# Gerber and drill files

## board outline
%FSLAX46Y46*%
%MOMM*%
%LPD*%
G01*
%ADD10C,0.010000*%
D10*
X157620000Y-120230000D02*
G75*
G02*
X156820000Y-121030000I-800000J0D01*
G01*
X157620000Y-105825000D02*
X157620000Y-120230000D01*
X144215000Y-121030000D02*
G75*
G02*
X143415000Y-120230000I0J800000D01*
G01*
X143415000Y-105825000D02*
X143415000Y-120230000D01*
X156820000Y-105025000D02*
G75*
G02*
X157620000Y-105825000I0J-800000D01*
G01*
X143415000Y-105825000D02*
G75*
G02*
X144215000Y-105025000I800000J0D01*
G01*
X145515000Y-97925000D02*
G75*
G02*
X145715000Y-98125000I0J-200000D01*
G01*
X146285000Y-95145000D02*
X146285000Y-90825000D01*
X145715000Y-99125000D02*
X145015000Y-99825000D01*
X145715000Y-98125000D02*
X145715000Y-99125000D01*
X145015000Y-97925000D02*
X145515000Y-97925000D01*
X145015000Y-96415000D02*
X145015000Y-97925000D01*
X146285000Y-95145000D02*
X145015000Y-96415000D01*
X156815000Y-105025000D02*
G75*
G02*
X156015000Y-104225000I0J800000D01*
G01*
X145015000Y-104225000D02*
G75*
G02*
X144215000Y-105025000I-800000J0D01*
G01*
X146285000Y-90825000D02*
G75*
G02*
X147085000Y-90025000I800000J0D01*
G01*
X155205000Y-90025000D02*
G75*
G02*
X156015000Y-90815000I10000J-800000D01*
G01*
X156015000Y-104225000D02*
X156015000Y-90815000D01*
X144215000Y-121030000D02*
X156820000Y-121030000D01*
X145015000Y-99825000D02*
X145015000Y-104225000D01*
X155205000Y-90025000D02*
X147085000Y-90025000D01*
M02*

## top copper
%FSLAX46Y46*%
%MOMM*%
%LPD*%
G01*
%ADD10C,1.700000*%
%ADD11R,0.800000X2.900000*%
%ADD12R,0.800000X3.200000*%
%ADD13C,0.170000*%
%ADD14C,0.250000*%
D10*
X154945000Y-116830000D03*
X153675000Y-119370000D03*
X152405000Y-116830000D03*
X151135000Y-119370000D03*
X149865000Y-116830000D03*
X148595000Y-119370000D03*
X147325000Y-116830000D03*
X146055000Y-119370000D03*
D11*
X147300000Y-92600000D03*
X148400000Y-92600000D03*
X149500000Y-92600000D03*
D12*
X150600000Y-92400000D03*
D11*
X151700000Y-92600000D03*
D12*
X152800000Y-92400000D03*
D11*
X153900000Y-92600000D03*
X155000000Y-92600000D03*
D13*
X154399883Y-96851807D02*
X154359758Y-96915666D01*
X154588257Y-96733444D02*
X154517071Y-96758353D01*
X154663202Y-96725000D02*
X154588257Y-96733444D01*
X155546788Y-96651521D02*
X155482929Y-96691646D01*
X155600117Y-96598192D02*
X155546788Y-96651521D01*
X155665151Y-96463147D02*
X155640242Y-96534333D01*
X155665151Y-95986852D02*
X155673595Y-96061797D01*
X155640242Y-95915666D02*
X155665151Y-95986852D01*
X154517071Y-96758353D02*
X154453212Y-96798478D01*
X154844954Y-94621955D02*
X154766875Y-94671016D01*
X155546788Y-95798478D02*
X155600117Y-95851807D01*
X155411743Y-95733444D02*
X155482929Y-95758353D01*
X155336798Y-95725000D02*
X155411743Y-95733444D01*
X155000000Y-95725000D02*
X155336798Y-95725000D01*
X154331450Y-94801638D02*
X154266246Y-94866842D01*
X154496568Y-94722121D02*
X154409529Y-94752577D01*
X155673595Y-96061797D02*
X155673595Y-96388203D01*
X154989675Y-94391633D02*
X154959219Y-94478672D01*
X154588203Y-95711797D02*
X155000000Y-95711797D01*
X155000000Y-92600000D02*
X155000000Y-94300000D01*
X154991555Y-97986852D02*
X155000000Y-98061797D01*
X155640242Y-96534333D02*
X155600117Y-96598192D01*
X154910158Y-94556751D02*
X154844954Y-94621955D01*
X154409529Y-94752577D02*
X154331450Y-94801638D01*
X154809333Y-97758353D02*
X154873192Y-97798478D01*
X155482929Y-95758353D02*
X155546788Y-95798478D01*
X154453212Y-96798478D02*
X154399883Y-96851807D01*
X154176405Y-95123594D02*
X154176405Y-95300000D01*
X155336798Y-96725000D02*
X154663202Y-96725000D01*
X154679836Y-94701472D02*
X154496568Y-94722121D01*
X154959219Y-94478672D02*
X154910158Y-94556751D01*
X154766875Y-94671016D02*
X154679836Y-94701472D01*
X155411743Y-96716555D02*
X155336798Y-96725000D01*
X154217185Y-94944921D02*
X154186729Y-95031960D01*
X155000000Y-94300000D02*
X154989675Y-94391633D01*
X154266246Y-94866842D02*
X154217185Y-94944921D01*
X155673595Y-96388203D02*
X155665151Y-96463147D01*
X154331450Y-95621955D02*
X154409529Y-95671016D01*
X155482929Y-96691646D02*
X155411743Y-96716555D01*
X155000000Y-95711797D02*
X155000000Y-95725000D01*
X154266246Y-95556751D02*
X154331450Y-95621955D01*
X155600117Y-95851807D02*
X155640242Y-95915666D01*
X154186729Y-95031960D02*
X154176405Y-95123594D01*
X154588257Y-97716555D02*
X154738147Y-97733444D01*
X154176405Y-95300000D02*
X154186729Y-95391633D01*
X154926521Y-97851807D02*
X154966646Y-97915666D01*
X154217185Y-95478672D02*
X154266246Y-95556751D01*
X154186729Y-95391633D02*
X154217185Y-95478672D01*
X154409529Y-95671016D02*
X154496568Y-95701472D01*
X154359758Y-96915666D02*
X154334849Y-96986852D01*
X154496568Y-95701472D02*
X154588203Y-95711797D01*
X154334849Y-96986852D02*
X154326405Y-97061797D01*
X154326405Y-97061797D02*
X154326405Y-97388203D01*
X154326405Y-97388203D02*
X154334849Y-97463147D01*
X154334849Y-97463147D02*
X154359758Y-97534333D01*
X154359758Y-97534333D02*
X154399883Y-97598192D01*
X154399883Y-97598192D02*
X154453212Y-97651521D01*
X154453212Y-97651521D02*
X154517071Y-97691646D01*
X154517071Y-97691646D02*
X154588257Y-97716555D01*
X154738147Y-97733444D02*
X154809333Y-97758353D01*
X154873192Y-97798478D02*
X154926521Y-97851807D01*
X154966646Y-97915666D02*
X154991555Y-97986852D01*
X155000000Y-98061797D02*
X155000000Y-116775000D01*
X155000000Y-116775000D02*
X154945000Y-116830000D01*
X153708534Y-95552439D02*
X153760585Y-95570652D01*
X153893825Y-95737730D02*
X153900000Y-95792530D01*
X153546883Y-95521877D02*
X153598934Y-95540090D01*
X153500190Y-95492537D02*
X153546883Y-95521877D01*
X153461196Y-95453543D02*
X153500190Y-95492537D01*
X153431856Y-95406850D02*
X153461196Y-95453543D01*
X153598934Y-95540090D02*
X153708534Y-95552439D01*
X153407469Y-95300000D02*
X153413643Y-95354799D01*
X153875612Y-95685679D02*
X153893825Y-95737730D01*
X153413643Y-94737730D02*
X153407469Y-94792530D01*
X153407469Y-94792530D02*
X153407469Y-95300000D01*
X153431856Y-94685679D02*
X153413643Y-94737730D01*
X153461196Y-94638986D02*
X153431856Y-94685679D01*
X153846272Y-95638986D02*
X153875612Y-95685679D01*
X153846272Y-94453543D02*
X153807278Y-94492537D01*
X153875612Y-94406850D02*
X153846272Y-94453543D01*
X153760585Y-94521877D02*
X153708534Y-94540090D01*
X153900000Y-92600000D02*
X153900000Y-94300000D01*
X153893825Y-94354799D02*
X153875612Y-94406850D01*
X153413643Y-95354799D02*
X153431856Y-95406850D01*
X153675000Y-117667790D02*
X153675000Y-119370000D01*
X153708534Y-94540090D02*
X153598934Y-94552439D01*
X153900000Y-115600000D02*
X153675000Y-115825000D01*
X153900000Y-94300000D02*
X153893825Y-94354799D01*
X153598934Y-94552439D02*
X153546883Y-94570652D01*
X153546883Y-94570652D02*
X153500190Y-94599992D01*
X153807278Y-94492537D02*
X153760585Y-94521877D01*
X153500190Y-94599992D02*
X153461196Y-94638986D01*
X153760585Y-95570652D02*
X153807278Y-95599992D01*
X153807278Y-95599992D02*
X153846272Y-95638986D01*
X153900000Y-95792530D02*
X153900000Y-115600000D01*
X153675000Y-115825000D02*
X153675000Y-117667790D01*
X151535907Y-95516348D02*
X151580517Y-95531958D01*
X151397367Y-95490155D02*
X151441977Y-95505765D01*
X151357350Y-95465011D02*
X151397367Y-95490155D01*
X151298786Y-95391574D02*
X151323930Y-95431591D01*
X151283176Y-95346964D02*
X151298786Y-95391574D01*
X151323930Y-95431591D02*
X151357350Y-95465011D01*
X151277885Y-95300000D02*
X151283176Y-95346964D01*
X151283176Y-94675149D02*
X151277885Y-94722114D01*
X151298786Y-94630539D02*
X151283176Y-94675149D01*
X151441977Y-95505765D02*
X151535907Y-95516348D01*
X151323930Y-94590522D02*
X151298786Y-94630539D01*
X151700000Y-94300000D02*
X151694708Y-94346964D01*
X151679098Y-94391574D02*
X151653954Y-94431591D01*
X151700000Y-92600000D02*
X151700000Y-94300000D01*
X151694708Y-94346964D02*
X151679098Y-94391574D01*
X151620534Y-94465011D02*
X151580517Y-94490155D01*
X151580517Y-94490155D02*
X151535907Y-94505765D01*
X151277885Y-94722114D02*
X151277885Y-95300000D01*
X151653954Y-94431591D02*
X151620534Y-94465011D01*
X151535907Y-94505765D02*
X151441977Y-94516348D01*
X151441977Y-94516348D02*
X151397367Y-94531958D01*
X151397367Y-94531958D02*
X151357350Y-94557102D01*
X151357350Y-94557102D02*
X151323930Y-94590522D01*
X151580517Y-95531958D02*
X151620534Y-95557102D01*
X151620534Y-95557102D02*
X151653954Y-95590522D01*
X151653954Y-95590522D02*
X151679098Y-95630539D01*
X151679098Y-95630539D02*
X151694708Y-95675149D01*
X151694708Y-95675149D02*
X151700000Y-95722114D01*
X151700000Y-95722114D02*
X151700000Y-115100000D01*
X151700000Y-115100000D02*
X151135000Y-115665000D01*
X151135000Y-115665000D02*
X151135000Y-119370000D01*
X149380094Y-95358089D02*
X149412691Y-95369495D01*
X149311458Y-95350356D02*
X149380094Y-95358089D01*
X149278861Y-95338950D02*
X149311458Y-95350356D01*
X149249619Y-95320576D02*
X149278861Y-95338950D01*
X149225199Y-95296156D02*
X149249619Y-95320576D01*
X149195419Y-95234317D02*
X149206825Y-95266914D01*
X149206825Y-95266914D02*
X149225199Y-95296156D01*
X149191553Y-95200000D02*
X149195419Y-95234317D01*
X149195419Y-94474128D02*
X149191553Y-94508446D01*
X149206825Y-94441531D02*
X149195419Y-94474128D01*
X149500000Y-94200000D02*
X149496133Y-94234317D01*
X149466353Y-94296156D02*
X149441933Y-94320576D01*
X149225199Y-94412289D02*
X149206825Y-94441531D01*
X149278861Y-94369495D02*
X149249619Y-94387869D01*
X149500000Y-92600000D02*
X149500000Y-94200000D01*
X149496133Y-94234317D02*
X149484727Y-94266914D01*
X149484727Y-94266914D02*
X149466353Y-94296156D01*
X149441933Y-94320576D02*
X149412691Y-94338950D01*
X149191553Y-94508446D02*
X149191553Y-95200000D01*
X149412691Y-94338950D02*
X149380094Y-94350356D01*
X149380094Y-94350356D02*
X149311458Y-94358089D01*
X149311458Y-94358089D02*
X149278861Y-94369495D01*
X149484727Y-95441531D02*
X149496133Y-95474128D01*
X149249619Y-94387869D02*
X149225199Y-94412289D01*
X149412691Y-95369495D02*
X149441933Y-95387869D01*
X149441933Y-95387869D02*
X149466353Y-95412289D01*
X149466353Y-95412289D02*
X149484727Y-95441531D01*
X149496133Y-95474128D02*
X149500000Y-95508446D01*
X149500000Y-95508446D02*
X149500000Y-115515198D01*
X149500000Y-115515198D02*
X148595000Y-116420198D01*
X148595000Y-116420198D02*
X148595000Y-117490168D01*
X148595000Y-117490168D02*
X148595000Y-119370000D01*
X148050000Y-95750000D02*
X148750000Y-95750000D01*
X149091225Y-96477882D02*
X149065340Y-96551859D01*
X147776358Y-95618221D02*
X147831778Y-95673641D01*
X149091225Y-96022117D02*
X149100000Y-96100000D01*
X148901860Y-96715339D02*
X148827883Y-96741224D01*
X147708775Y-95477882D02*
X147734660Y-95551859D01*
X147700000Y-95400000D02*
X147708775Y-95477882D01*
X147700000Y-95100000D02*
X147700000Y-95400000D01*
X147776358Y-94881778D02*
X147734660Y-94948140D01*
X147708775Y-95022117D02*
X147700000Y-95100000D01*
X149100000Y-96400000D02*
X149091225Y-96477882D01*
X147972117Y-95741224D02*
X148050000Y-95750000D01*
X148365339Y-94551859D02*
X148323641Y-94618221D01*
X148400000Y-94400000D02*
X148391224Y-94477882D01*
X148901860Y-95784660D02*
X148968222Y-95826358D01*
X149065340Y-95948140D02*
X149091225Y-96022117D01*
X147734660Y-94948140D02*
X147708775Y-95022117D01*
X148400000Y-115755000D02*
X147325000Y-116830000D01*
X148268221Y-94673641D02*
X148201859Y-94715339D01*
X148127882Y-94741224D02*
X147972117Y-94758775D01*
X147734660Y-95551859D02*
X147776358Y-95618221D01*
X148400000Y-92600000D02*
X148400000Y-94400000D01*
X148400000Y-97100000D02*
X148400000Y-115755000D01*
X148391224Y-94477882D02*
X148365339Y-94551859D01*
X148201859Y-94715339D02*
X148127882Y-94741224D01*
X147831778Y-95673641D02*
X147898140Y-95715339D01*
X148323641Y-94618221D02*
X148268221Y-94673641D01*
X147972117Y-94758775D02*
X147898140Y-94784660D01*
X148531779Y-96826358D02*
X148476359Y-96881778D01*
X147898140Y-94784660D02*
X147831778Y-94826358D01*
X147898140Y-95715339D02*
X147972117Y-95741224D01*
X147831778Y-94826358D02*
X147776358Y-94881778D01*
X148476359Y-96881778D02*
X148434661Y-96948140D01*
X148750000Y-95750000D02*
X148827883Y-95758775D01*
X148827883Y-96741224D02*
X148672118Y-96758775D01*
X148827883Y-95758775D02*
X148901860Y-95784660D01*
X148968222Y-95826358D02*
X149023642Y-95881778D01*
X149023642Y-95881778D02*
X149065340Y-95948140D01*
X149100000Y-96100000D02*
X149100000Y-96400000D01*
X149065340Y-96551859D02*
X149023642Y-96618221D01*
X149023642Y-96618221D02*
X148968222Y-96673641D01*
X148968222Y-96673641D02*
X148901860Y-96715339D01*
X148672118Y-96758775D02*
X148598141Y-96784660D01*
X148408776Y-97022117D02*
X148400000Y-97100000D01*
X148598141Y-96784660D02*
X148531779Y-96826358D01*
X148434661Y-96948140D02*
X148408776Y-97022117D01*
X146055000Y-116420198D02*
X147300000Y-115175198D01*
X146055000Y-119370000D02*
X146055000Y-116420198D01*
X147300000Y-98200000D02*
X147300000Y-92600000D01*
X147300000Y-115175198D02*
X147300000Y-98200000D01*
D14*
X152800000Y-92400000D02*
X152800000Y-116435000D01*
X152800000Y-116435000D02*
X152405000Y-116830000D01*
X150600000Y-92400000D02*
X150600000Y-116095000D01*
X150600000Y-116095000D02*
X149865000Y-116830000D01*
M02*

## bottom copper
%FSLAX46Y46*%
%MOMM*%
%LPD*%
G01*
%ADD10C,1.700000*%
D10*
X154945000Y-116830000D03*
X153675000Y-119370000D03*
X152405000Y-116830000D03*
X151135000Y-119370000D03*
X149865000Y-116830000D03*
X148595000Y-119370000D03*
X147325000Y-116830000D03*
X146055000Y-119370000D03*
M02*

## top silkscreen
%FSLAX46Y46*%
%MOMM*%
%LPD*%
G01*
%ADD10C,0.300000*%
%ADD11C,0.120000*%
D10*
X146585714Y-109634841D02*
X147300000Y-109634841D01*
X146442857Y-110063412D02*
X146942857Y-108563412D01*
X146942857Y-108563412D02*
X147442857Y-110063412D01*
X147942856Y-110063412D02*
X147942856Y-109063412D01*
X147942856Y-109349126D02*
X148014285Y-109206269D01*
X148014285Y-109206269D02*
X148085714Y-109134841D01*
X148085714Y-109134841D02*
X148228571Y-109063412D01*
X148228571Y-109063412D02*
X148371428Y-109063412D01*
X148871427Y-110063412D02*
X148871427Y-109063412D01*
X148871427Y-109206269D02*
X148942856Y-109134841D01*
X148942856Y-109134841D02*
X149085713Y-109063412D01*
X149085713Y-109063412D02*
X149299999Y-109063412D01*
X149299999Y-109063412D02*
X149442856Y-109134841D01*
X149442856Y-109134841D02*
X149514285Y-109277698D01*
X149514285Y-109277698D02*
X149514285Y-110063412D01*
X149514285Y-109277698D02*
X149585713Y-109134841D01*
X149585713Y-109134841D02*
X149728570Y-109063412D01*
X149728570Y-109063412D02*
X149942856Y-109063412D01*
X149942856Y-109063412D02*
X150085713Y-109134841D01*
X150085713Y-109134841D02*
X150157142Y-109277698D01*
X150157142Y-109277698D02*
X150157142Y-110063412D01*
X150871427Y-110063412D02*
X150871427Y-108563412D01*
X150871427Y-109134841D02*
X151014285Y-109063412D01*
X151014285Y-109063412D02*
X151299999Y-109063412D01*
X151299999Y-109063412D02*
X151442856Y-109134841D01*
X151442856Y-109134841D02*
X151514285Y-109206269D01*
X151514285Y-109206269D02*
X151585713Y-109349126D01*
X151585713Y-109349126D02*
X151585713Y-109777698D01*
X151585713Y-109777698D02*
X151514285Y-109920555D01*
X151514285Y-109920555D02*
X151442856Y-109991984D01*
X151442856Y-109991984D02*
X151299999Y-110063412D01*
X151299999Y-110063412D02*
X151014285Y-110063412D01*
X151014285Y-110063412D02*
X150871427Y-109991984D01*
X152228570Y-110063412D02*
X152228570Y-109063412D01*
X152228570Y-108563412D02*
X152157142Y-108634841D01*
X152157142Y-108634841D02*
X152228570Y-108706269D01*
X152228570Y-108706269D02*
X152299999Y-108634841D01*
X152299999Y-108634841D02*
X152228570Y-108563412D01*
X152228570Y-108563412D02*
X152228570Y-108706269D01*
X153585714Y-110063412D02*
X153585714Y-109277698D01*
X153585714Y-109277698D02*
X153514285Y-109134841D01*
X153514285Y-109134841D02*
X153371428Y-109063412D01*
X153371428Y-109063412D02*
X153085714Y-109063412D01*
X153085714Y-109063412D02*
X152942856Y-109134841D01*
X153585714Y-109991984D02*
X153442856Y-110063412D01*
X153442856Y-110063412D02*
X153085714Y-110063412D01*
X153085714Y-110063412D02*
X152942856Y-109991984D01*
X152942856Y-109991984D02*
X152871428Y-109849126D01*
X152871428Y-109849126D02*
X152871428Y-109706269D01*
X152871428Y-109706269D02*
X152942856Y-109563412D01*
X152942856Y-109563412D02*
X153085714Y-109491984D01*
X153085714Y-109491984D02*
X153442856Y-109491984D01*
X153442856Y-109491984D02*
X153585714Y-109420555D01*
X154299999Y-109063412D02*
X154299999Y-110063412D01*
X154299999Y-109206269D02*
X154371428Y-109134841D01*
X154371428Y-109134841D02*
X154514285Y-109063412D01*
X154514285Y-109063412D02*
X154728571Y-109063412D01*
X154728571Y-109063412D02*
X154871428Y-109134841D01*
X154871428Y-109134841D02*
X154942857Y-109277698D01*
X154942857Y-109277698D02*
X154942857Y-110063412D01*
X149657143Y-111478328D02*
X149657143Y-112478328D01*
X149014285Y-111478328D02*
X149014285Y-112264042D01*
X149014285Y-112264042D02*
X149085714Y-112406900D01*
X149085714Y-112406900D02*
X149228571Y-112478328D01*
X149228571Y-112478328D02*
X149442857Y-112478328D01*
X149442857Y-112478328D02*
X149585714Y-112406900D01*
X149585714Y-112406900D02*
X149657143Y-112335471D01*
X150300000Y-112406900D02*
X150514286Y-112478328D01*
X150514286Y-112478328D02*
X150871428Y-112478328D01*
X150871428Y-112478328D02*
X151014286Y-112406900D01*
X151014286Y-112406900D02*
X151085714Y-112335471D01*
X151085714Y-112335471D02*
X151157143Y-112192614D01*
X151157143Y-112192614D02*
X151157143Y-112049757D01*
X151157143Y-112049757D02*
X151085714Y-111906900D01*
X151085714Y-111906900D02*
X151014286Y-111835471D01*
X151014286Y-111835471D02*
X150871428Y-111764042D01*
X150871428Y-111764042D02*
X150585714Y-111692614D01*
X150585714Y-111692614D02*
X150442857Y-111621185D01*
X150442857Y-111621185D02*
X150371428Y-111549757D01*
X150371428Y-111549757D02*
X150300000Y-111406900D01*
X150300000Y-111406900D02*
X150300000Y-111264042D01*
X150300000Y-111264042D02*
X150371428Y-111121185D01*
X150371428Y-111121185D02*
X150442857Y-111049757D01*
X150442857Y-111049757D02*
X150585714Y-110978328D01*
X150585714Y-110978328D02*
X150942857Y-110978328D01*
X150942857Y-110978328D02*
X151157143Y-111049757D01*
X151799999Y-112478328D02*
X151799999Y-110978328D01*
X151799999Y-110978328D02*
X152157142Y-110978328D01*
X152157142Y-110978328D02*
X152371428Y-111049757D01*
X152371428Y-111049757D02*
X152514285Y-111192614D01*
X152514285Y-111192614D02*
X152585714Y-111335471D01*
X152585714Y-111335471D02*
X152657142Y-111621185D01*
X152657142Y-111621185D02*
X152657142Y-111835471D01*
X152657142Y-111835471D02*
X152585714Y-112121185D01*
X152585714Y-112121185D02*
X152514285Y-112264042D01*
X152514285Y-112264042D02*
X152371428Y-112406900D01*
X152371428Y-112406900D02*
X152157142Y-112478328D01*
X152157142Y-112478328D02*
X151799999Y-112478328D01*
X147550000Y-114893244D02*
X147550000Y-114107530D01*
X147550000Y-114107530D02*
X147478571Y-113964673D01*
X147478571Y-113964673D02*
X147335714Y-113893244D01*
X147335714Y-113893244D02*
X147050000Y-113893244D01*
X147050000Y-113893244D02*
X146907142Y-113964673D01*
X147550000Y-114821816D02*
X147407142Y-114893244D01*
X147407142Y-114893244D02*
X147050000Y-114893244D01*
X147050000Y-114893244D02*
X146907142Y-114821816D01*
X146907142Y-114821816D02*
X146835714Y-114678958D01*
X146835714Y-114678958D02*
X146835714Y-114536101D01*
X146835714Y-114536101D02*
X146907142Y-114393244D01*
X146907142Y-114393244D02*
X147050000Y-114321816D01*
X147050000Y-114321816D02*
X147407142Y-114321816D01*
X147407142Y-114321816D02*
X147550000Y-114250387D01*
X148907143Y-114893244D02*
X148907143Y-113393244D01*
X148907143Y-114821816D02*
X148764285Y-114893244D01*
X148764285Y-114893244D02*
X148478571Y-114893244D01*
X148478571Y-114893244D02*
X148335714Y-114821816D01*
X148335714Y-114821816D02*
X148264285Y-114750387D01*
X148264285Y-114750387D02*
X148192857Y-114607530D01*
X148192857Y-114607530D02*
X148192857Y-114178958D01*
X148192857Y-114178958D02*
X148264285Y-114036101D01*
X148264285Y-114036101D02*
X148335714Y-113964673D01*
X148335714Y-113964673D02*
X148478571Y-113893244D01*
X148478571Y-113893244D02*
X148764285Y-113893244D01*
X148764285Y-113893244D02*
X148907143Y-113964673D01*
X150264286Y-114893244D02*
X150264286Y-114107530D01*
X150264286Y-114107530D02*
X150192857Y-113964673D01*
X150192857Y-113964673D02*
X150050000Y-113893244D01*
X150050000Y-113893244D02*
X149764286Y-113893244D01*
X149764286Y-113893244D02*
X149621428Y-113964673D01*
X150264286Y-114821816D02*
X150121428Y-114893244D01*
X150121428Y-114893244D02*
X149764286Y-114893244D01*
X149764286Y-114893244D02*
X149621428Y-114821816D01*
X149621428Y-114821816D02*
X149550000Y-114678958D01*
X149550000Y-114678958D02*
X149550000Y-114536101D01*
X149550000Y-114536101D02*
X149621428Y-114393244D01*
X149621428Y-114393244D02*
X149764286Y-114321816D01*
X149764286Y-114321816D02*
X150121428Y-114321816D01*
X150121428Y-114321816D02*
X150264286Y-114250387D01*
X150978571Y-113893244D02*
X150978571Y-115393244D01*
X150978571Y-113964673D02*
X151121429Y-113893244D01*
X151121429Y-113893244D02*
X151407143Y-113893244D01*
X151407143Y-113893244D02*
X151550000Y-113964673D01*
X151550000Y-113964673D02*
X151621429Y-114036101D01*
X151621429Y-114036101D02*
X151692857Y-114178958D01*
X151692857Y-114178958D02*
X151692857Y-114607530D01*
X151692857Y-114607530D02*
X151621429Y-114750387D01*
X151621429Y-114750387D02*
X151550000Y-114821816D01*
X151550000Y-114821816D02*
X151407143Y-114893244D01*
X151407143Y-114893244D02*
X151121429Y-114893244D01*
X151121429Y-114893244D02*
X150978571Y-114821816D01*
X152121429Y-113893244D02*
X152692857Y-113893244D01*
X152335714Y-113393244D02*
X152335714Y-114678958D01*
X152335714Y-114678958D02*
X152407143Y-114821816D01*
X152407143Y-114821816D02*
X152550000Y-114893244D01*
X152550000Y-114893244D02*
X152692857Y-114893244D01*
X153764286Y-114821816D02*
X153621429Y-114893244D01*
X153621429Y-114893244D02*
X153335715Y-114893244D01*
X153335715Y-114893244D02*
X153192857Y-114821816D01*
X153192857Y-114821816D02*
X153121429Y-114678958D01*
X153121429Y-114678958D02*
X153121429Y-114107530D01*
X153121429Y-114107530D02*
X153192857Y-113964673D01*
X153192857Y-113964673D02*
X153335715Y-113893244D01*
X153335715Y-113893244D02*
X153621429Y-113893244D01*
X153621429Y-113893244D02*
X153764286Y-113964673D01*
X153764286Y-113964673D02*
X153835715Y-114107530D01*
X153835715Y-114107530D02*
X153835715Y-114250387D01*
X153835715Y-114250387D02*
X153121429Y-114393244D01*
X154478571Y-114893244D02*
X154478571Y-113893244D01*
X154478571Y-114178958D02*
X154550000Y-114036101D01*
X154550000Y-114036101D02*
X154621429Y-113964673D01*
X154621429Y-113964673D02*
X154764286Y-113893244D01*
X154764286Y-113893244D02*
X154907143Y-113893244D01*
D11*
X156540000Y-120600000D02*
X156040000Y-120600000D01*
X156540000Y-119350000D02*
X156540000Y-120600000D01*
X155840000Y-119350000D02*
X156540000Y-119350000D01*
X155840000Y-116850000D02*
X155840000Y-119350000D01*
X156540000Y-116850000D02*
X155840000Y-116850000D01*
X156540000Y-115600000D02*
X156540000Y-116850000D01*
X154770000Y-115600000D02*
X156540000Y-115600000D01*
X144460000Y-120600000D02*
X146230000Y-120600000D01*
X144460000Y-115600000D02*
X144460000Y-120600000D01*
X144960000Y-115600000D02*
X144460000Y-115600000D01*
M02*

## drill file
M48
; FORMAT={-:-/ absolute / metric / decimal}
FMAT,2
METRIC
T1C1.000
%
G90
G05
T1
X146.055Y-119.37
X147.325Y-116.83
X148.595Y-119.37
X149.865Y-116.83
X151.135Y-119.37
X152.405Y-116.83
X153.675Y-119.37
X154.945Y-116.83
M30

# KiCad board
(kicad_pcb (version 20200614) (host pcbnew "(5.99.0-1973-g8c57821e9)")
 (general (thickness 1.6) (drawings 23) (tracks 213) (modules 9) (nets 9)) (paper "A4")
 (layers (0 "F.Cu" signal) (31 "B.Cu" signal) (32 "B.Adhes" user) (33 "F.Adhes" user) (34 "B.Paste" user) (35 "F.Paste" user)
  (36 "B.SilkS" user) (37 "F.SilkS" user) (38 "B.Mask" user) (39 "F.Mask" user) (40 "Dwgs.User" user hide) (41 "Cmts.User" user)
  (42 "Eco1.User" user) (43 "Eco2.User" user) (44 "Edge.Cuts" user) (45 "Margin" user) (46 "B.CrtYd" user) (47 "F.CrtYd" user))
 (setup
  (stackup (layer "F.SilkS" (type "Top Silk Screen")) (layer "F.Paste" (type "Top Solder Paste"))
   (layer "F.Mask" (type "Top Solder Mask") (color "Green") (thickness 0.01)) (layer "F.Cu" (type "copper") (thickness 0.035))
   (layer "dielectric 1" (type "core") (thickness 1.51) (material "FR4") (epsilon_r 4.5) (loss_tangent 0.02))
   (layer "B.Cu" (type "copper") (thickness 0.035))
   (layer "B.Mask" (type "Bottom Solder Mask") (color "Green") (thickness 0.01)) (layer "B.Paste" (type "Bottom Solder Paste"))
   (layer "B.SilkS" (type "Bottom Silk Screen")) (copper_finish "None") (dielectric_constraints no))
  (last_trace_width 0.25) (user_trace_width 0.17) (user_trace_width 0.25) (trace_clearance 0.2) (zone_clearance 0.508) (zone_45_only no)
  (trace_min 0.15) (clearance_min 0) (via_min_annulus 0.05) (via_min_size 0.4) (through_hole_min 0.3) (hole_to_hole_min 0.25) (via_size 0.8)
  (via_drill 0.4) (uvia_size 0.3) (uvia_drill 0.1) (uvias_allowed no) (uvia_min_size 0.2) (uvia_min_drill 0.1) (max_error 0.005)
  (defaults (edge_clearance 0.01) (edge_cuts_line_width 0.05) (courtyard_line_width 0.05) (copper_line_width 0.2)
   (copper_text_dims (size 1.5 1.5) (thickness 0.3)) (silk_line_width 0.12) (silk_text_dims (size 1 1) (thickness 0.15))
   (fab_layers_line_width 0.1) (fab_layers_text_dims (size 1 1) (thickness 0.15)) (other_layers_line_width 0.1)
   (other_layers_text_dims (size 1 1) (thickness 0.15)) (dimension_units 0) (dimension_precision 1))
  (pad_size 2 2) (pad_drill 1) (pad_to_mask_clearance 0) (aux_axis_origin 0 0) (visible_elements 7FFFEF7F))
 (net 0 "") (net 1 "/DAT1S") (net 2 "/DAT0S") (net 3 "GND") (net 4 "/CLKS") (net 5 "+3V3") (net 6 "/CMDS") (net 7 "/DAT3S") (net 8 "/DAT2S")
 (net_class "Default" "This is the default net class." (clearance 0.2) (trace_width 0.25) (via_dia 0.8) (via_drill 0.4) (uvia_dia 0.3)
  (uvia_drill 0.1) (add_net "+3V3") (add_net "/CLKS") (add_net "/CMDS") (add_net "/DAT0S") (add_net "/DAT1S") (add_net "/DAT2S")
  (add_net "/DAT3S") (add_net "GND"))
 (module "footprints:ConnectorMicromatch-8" (layer "F.Cu") (at 150.5 118.1)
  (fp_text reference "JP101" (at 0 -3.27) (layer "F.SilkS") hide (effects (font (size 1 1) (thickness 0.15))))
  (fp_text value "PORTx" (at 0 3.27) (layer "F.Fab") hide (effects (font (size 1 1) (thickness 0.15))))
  (fp_line (start 6.04 2.5) (end 5.54 2.5) (layer "F.SilkS") (width 0.12))
  (fp_line (start 6.04 1.25) (end 6.04 2.5) (layer "F.SilkS") (width 0.12))
  (fp_line (start 5.34 1.25) (end 6.04 1.25) (layer "F.SilkS") (width 0.12))
  (fp_line (start 5.34 -1.25) (end 5.34 1.25) (layer "F.SilkS") (width 0.12))
  (fp_line (start 6.04 -1.25) (end 5.34 -1.25) (layer "F.SilkS") (width 0.12))
  (fp_line (start 6.04 -2.5) (end 6.04 -1.25) (layer "F.SilkS") (width 0.12))
  (fp_line (start 4.27 -2.5) (end 6.04 -2.5) (layer "F.SilkS") (width 0.12))
  (fp_line (start -6.04 2.5) (end -4.27 2.5) (layer "F.SilkS") (width 0.12))
  (fp_line (start -6.04 -2.5) (end -6.04 2.5) (layer "F.SilkS") (width 0.12))
  (fp_line (start -5.54 -2.5) (end -6.04 -2.5) (layer "F.SilkS") (width 0.12))
  (pad "8" thru_hole circle (at 4.445 -1.27) (size 1.7 1.7) (drill 1) (layers *.Cu *.Mask) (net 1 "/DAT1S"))
  (pad "7" thru_hole circle (at 3.175 1.27) (size 1.7 1.7) (drill 1) (layers *.Cu *.Mask) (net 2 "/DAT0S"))
  (pad "6" thru_hole circle (at 1.905 -1.27) (size 1.7 1.7) (drill 1) (layers *.Cu *.Mask) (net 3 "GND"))
  (pad "5" thru_hole circle (at 0.635 1.27) (size 1.7 1.7) (drill 1) (layers *.Cu *.Mask) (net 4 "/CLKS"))
  (pad "4" thru_hole circle (at -0.635 -1.27) (size 1.7 1.7) (drill 1) (layers *.Cu *.Mask) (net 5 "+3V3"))
  (pad "3" thru_hole circle (at -1.905 1.27) (size 1.7 1.7) (drill 1) (layers *.Cu *.Mask) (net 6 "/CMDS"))
  (pad "2" thru_hole circle (at -3.175 -1.27) (size 1.7 1.7) (drill 1) (layers *.Cu *.Mask) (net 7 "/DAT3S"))
  (pad "1" thru_hole circle (at -4.445 1.27) (size 1.7 1.7) (drill 1) (layers *.Cu *.Mask) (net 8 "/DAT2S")))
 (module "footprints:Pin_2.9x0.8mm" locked (layer "F.Cu") (at 147.3 92.6)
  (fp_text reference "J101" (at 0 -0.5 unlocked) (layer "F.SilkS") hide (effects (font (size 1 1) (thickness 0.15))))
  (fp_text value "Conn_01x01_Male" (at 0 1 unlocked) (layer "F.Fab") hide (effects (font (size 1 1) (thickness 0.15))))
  (pad "1" smd rect (at 0 0) (size 0.8 2.9) (layers "F.Cu" "F.Paste" "F.Mask") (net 8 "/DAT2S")))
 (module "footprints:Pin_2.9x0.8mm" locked (layer "F.Cu") (at 148.4 92.6)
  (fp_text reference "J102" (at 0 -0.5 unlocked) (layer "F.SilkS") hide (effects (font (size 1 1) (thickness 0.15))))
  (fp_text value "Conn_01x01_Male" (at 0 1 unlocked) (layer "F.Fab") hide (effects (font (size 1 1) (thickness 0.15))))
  (pad "1" smd rect (at 0 0) (size 0.8 2.9) (layers "F.Cu" "F.Paste" "F.Mask") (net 7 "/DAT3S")))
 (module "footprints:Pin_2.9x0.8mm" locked (layer "F.Cu") (at 149.5 92.6)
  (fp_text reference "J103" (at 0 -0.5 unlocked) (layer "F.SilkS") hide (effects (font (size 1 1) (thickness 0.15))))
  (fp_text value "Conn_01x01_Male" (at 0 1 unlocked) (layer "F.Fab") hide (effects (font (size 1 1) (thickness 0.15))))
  (pad "1" smd rect (at 0 0) (size 0.8 2.9) (layers "F.Cu" "F.Paste" "F.Mask") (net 6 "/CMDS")))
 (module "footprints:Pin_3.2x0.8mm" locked (layer "F.Cu") (at 150.6 92.4)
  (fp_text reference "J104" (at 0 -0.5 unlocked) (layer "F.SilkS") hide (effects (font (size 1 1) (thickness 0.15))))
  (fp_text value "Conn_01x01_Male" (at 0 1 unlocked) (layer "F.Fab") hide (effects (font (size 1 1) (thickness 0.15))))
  (pad "1" smd rect (at 0 0) (size 0.8 3.2) (layers "F.Cu" "F.Paste" "F.Mask") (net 5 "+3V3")))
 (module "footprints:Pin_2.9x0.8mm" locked (layer "F.Cu") (at 151.7 92.6)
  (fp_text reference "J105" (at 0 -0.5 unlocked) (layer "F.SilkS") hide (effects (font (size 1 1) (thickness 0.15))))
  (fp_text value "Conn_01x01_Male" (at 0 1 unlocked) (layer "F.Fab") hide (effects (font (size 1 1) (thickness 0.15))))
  (pad "1" smd rect (at 0 0) (size 0.8 2.9) (layers "F.Cu" "F.Paste" "F.Mask") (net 4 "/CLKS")))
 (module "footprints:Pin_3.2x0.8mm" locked (layer "F.Cu") (at 152.8 92.4)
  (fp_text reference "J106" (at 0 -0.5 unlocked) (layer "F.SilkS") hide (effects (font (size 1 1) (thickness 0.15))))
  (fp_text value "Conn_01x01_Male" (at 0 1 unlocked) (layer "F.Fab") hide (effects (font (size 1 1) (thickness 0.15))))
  (pad "1" smd rect (at 0 0) (size 0.8 3.2) (layers "F.Cu" "F.Paste" "F.Mask") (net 3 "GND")))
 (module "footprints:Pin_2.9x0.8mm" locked (layer "F.Cu") (at 153.9 92.6)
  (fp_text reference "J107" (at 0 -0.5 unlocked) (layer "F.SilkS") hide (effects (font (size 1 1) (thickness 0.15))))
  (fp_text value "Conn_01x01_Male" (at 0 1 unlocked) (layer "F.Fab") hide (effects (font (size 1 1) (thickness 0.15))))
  (pad "1" smd rect (at 0 0) (size 0.8 2.9) (layers "F.Cu" "F.Paste" "F.Mask") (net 2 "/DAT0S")))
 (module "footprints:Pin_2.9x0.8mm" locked (layer "F.Cu") (at 155 92.6)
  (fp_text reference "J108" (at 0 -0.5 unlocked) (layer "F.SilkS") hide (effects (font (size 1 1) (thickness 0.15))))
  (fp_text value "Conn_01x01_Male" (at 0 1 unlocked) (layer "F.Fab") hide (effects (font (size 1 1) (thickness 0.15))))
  (pad "1" smd rect (at 0 0) (size 0.8 2.9) (layers "F.Cu" "F.Paste" "F.Mask") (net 1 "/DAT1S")))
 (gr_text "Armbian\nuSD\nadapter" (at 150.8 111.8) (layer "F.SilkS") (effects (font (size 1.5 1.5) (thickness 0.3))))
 (gr_arc (start 156.82 120.23) (end 157.62 120.23) (angle 90) (layer "Edge.Cuts") (width 0.01))
 (gr_line (start 157.62 105.825) (end 157.62 120.23) (layer "Edge.Cuts") (width 0.01))
 (gr_arc (start 144.215 120.23) (end 144.215 121.03) (angle 90) (layer "Edge.Cuts") (width 0.01))
 (gr_line (start 143.415 105.825) (end 143.415 120.23) (layer "Edge.Cuts") (width 0.01))
 (gr_arc (start 156.82 105.825) (end 156.82 105.025) (angle 90) (layer "Edge.Cuts") (width 0.01))
 (gr_arc (start 144.215 105.825) (end 143.415 105.825) (angle 90) (layer "Edge.Cuts") (width 0.01))
 (gr_arc (start 145.515 98.125) (end 145.515 97.925) (angle 90) (layer "Edge.Cuts") (width 0.01))
 (gr_line (start 146.285 95.145) (end 146.285 90.825) (layer "Edge.Cuts") (width 0.01))
 (gr_line (start 145.715 99.125) (end 145.015 99.825) (layer "Edge.Cuts") (width 0.01))
 (gr_line (start 145.715 98.125) (end 145.715 99.125) (layer "Edge.Cuts") (width 0.01))
 (gr_line (start 145.015 97.925) (end 145.515 97.925) (layer "Edge.Cuts") (width 0.01))
 (gr_line (start 145.015 96.415) (end 145.015 97.925) (layer "Edge.Cuts") (width 0.01))
 (gr_line (start 146.285 95.145) (end 145.015 96.415) (layer "Edge.Cuts") (width 0.01))
 (gr_arc (start 156.815 104.225) (end 156.815 105.025) (angle 90) (layer "Edge.Cuts") (width 0.01))
 (gr_arc (start 144.215 104.225) (end 145.015 104.225) (angle 90) (layer "Edge.Cuts") (width 0.01))
 (gr_arc (start 147.085 90.825) (end 146.285 90.825) (angle 90) (layer "Edge.Cuts") (width 0.01))
 (gr_arc (start 155.215 90.825) (end 155.205 90.025) (angle 90) (layer "Edge.Cuts") (width 0.01))
 (gr_line (start 156.015 104.225) (end 156.015 90.815) (layer "Edge.Cuts") (width 0.01))
 (gr_line (start 144.215 121.03) (end 156.82 121.03) (layer "Edge.Cuts") (width 0.01))
 (gr_line (start 145.015 99.825) (end 145.015 104.225) (layer "Edge.Cuts") (width 0.01))
 (gr_line (start 155.205 90.025) (end 147.085 90.025) (layer "Edge.Cuts") (width 0.01))
 (segment (start 154.399883 96.851807) (end 154.359758 96.915666) (width 0.17) (layer "F.Cu") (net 1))
 (segment (start 154.588257 96.733444) (end 154.517071 96.758353) (width 0.17) (layer "F.Cu") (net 1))
 (segment (start 154.663202 96.725) (end 154.588257 96.733444) (width 0.17) (layer "F.Cu") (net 1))
 (segment (start 155.546788 96.651521) (end 155.482929 96.691646) (width 0.17) (layer "F.Cu") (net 1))
 (segment (start 155.600117 96.598192) (end 155.546788 96.651521) (width 0.17) (layer "F.Cu") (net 1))
 (segment (start 155.665151 96.463147) (end 155.640242 96.534333) (width 0.17) (layer "F.Cu") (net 1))
 (segment (start 155.665151 95.986852) (end 155.673595 96.061797) (width 0.17) (layer "F.Cu") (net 1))
 (segment (start 155.640242 95.915666) (end 155.665151 95.986852) (width 0.17) (layer "F.Cu") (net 1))
 (segment (start 154.517071 96.758353) (end 154.453212 96.798478) (width 0.17) (layer "F.Cu") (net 1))
 (segment (start 154.844954 94.621955) (end 154.766875 94.671016) (width 0.17) (layer "F.Cu") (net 1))
 (segment (start 155.546788 95.798478) (end 155.600117 95.851807) (width 0.17) (layer "F.Cu") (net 1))
 (segment (start 155.411743 95.733444) (end 155.482929 95.758353) (width 0.17) (layer "F.Cu") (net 1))
 (segment (start 155.336798 95.725) (end 155.411743 95.733444) (width 0.17) (layer "F.Cu") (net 1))
 (segment (start 155 95.725) (end 155.336798 95.725) (width 0.17) (layer "F.Cu") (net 1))
 (segment (start 154.33145 94.801638) (end 154.266246 94.866842) (width 0.17) (layer "F.Cu") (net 1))
 (segment (start 154.496568 94.722121) (end 154.409529 94.752577) (width 0.17) (layer "F.Cu") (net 1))
 (segment (start 155.673595 96.061797) (end 155.673595 96.388203) (width 0.17) (layer "F.Cu") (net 1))
 (segment (start 154.989675 94.391633) (end 154.959219 94.478672) (width 0.17) (layer "F.Cu") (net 1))
 (segment (start 154.588203 95.711797) (end 155 95.711797) (width 0.17) (layer "F.Cu") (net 1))
 (segment (start 155 92.6) (end 155 94.3) (width 0.17) (layer "F.Cu") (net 1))
 (segment (start 154.991555 97.986852) (end 155 98.061797) (width 0.17) (layer "F.Cu") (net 1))
 (segment (start 155.640242 96.534333) (end 155.600117 96.598192) (width 0.17) (layer "F.Cu") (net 1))
 (segment (start 154.910158 94.556751) (end 154.844954 94.621955) (width 0.17) (layer "F.Cu") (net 1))
 (segment (start 154.409529 94.752577) (end 154.33145 94.801638) (width 0.17) (layer "F.Cu") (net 1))
 (segment (start 154.809333 97.758353) (end 154.873192 97.798478) (width 0.17) (layer "F.Cu") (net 1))
 (segment (start 155.482929 95.758353) (end 155.546788 95.798478) (width 0.17) (layer "F.Cu") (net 1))
 (segment (start 154.453212 96.798478) (end 154.399883 96.851807) (width 0.17) (layer "F.Cu") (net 1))
 (segment (start 154.176405 95.123594) (end 154.176405 95.3) (width 0.17) (layer "F.Cu") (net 1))
 (segment (start 155.336798 96.725) (end 154.663202 96.725) (width 0.17) (layer "F.Cu") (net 1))
 (segment (start 154.679836 94.701472) (end 154.496568 94.722121) (width 0.17) (layer "F.Cu") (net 1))
 (segment (start 154.959219 94.478672) (end 154.910158 94.556751) (width 0.17) (layer "F.Cu") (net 1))
 (segment (start 154.766875 94.671016) (end 154.679836 94.701472) (width 0.17) (layer "F.Cu") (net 1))
 (segment (start 155.411743 96.716555) (end 155.336798 96.725) (width 0.17) (layer "F.Cu") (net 1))
 (segment (start 154.217185 94.944921) (end 154.186729 95.03196) (width 0.17) (layer "F.Cu") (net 1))
 (segment (start 155 94.3) (end 154.989675 94.391633) (width 0.17) (layer "F.Cu") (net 1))
 (segment (start 154.266246 94.866842) (end 154.217185 94.944921) (width 0.17) (layer "F.Cu") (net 1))
 (segment (start 155.673595 96.388203) (end 155.665151 96.463147) (width 0.17) (layer "F.Cu") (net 1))
 (segment (start 154.33145 95.621955) (end 154.409529 95.671016) (width 0.17) (layer "F.Cu") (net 1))
 (segment (start 155.482929 96.691646) (end 155.411743 96.716555) (width 0.17) (layer "F.Cu") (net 1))
 (segment (start 155 95.711797) (end 155 95.725) (width 0.17) (layer "F.Cu") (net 1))
 (segment (start 154.266246 95.556751) (end 154.33145 95.621955) (width 0.17) (layer "F.Cu") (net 1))
 (segment (start 155.600117 95.851807) (end 155.640242 95.915666) (width 0.17) (layer "F.Cu") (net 1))
 (segment (start 154.186729 95.03196) (end 154.176405 95.123594) (width 0.17) (layer "F.Cu") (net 1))
 (segment (start 154.588257 97.716555) (end 154.738147 97.733444) (width 0.17) (layer "F.Cu") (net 1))
 (segment (start 154.176405 95.3) (end 154.186729 95.391633) (width 0.17) (layer "F.Cu") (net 1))
 (segment (start 154.926521 97.851807) (end 154.966646 97.915666) (width 0.17) (layer "F.Cu") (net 1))
 (segment (start 154.217185 95.478672) (end 154.266246 95.556751) (width 0.17) (layer "F.Cu") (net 1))
 (segment (start 154.186729 95.391633) (end 154.217185 95.478672) (width 0.17) (layer "F.Cu") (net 1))
 (segment (start 154.409529 95.671016) (end 154.496568 95.701472) (width 0.17) (layer "F.Cu") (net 1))
 (segment (start 154.359758 96.915666) (end 154.334849 96.986852) (width 0.17) (layer "F.Cu") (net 1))
 (segment (start 154.496568 95.701472) (end 154.588203 95.711797) (width 0.17) (layer "F.Cu") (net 1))
 (segment (start 154.334849 96.986852) (end 154.326405 97.061797) (width 0.17) (layer "F.Cu") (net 1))
 (segment (start 154.326405 97.061797) (end 154.326405 97.388203) (width 0.17) (layer "F.Cu") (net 1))
 (segment (start 154.326405 97.388203) (end 154.334849 97.463147) (width 0.17) (layer "F.Cu") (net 1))
 (segment (start 154.334849 97.463147) (end 154.359758 97.534333) (width 0.17) (layer "F.Cu") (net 1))
 (segment (start 154.359758 97.534333) (end 154.399883 97.598192) (width 0.17) (layer "F.Cu") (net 1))
 (segment (start 154.399883 97.598192) (end 154.453212 97.651521) (width 0.17) (layer "F.Cu") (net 1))
 (segment (start 154.453212 97.651521) (end 154.517071 97.691646) (width 0.17) (layer "F.Cu") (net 1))
 (segment (start 154.517071 97.691646) (end 154.588257 97.716555) (width 0.17) (layer "F.Cu") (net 1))
 (segment (start 154.738147 97.733444) (end 154.809333 97.758353) (width 0.17) (layer "F.Cu") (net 1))
 (segment (start 154.873192 97.798478) (end 154.926521 97.851807) (width 0.17) (layer "F.Cu") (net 1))
 (segment (start 154.966646 97.915666) (end 154.991555 97.986852) (width 0.17) (layer "F.Cu") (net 1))
 (segment (start 155 98.061797) (end 155 116.775) (width 0.17) (layer "F.Cu") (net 1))
 (segment (start 155 116.775) (end 154.945 116.83) (width 0.17) (layer "F.Cu") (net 1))
 (segment (start 153.708534 95.552439) (end 153.760585 95.570652) (width 0.17) (layer "F.Cu") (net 2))
 (segment (start 153.893825 95.73773) (end 153.9 95.79253) (width 0.17) (layer "F.Cu") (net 2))
 (segment (start 153.546883 95.521877) (end 153.598934 95.54009) (width 0.17) (layer "F.Cu") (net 2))
 (segment (start 153.50019 95.492537) (end 153.546883 95.521877) (width 0.17) (layer "F.Cu") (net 2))
 (segment (start 153.461196 95.453543) (end 153.50019 95.492537) (width 0.17) (layer "F.Cu") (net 2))
 (segment (start 153.431856 95.40685) (end 153.461196 95.453543) (width 0.17) (layer "F.Cu") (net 2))
 (segment (start 153.598934 95.54009) (end 153.708534 95.552439) (width 0.17) (layer "F.Cu") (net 2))
 (segment (start 153.407469 95.3) (end 153.413643 95.354799) (width 0.17) (layer "F.Cu") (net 2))
 (segment (start 153.875612 95.685679) (end 153.893825 95.73773) (width 0.17) (layer "F.Cu") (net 2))
 (segment (start 153.413643 94.73773) (end 153.407469 94.79253) (width 0.17) (layer "F.Cu") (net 2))
 (segment (start 153.407469 94.79253) (end 153.407469 95.3) (width 0.17) (layer "F.Cu") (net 2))
 (segment (start 153.431856 94.685679) (end 153.413643 94.73773) (width 0.17) (layer "F.Cu") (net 2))
 (segment (start 153.461196 94.638986) (end 153.431856 94.685679) (width 0.17) (layer "F.Cu") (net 2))
 (segment (start 153.846272 95.638986) (end 153.875612 95.685679) (width 0.17) (layer "F.Cu") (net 2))
 (segment (start 153.846272 94.453543) (end 153.807278 94.492537) (width 0.17) (layer "F.Cu") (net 2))
 (segment (start 153.875612 94.40685) (end 153.846272 94.453543) (width 0.17) (layer "F.Cu") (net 2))
 (segment (start 153.760585 94.521877) (end 153.708534 94.54009) (width 0.17) (layer "F.Cu") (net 2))
 (segment (start 153.9 92.6) (end 153.9 94.3) (width 0.17) (layer "F.Cu") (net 2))
 (segment (start 153.893825 94.354799) (end 153.875612 94.40685) (width 0.17) (layer "F.Cu") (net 2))
 (segment (start 153.413643 95.354799) (end 153.431856 95.40685) (width 0.17) (layer "F.Cu") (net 2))
 (segment (start 153.675 117.66779) (end 153.675 119.37) (width 0.17) (layer "F.Cu") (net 2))
 (segment (start 153.708534 94.54009) (end 153.598934 94.552439) (width 0.17) (layer "F.Cu") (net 2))
 (segment (start 153.9 115.6) (end 153.675 115.825) (width 0.17) (layer "F.Cu") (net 2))
 (segment (start 153.9 94.3) (end 153.893825 94.354799) (width 0.17) (layer "F.Cu") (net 2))
 (segment (start 153.598934 94.552439) (end 153.546883 94.570652) (width 0.17) (layer "F.Cu") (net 2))
 (segment (start 153.546883 94.570652) (end 153.50019 94.599992) (width 0.17) (layer "F.Cu") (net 2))
 (segment (start 153.807278 94.492537) (end 153.760585 94.521877) (width 0.17) (layer "F.Cu") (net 2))
 (segment (start 153.50019 94.599992) (end 153.461196 94.638986) (width 0.17) (layer "F.Cu") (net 2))
 (segment (start 153.760585 95.570652) (end 153.807278 95.599992) (width 0.17) (layer "F.Cu") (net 2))
 (segment (start 153.807278 95.599992) (end 153.846272 95.638986) (width 0.17) (layer "F.Cu") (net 2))
 (segment (start 153.9 95.79253) (end 153.9 115.6) (width 0.17) (layer "F.Cu") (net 2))
 (segment (start 153.675 115.825) (end 153.675 117.66779) (width 0.17) (layer "F.Cu") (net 2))
 (segment (start 151.535907 95.516348) (end 151.580517 95.531958) (width 0.17) (layer "F.Cu") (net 4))
 (segment (start 151.397367 95.490155) (end 151.441977 95.505765) (width 0.17) (layer "F.Cu") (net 4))
 (segment (start 151.35735 95.465011) (end 151.397367 95.490155) (width 0.17) (layer "F.Cu") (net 4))
 (segment (start 151.298786 95.391574) (end 151.32393 95.431591) (width 0.17) (layer "F.Cu") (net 4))
 (segment (start 151.283176 95.346964) (end 151.298786 95.391574) (width 0.17) (layer "F.Cu") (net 4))
 (segment (start 151.32393 95.431591) (end 151.35735 95.465011) (width 0.17) (layer "F.Cu") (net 4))
 (segment (start 151.277885 95.3) (end 151.283176 95.346964) (width 0.17) (layer "F.Cu") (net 4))
 (segment (start 151.283176 94.675149) (end 151.277885 94.722114) (width 0.17) (layer "F.Cu") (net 4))
 (segment (start 151.298786 94.630539) (end 151.283176 94.675149) (width 0.17) (layer "F.Cu") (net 4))
 (segment (start 151.441977 95.505765) (end 151.535907 95.516348) (width 0.17) (layer "F.Cu") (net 4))
 (segment (start 151.32393 94.590522) (end 151.298786 94.630539) (width 0.17) (layer "F.Cu") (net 4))
 (segment (start 151.7 94.3) (end 151.694708 94.346964) (width 0.17) (layer "F.Cu") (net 4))
 (segment (start 151.679098 94.391574) (end 151.653954 94.431591) (width 0.17) (layer "F.Cu") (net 4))
 (segment (start 151.7 92.6) (end 151.7 94.3) (width 0.17) (layer "F.Cu") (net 4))
 (segment (start 151.694708 94.346964) (end 151.679098 94.391574) (width 0.17) (layer "F.Cu") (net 4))
 (segment (start 151.620534 94.465011) (end 151.580517 94.490155) (width 0.17) (layer "F.Cu") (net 4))
 (segment (start 151.580517 94.490155) (end 151.535907 94.505765) (width 0.17) (layer "F.Cu") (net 4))
 (segment (start 151.277885 94.722114) (end 151.277885 95.3) (width 0.17) (layer "F.Cu") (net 4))
 (segment (start 151.653954 94.431591) (end 151.620534 94.465011) (width 0.17) (layer "F.Cu") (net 4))
 (segment (start 151.535907 94.505765) (end 151.441977 94.516348) (width 0.17) (layer "F.Cu") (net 4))
 (segment (start 151.441977 94.516348) (end 151.397367 94.531958) (width 0.17) (layer "F.Cu") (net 4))
 (segment (start 151.397367 94.531958) (end 151.35735 94.557102) (width 0.17) (layer "F.Cu") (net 4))
 (segment (start 151.35735 94.557102) (end 151.32393 94.590522) (width 0.17) (layer "F.Cu") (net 4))
 (segment (start 151.580517 95.531958) (end 151.620534 95.557102) (width 0.17) (layer "F.Cu") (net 4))
 (segment (start 151.620534 95.557102) (end 151.653954 95.590522) (width 0.17) (layer "F.Cu") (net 4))
 (segment (start 151.653954 95.590522) (end 151.679098 95.630539) (width 0.17) (layer "F.Cu") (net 4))
 (segment (start 151.679098 95.630539) (end 151.694708 95.675149) (width 0.17) (layer "F.Cu") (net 4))
 (segment (start 151.694708 95.675149) (end 151.7 95.722114) (width 0.17) (layer "F.Cu") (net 4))
 (segment (start 151.7 95.722114) (end 151.7 115.1) (width 0.17) (layer "F.Cu") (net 4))
 (segment (start 151.7 115.1) (end 151.135 115.665) (width 0.17) (layer "F.Cu") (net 4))
 (segment (start 151.135 115.665) (end 151.135 119.37) (width 0.17) (layer "F.Cu") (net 4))
 (segment (start 149.380094 95.358089) (end 149.412691 95.369495) (width 0.17) (layer "F.Cu") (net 6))
 (segment (start 149.311458 95.350356) (end 149.380094 95.358089) (width 0.17) (layer "F.Cu") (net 6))
 (segment (start 149.278861 95.33895) (end 149.311458 95.350356) (width 0.17) (layer "F.Cu") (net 6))
 (segment (start 149.249619 95.320576) (end 149.278861 95.33895) (width 0.17) (layer "F.Cu") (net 6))
 (segment (start 149.225199 95.296156) (end 149.249619 95.320576) (width 0.17) (layer "F.Cu") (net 6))
 (segment (start 149.195419 95.234317) (end 149.206825 95.266914) (width 0.17) (layer "F.Cu") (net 6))
 (segment (start 149.206825 95.266914) (end 149.225199 95.296156) (width 0.17) (layer "F.Cu") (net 6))
 (segment (start 149.191553 95.2) (end 149.195419 95.234317) (width 0.17) (layer "F.Cu") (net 6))
 (segment (start 149.195419 94.474128) (end 149.191553 94.508446) (width 0.17) (layer "F.Cu") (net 6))
 (segment (start 149.206825 94.441531) (end 149.195419 94.474128) (width 0.17) (layer "F.Cu") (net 6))
 (segment (start 149.5 94.2) (end 149.496133 94.234317) (width 0.17) (layer "F.Cu") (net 6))
 (segment (start 149.466353 94.296156) (end 149.441933 94.320576) (width 0.17) (layer "F.Cu") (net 6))
 (segment (start 149.225199 94.412289) (end 149.206825 94.441531) (width 0.17) (layer "F.Cu") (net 6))
 (segment (start 149.278861 94.369495) (end 149.249619 94.387869) (width 0.17) (layer "F.Cu") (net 6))
 (segment (start 149.5 92.6) (end 149.5 94.2) (width 0.17) (layer "F.Cu") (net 6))
 (segment (start 149.496133 94.234317) (end 149.484727 94.266914) (width 0.17) (layer "F.Cu") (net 6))
 (segment (start 149.484727 94.266914) (end 149.466353 94.296156) (width 0.17) (layer "F.Cu") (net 6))
 (segment (start 149.441933 94.320576) (end 149.412691 94.33895) (width 0.17) (layer "F.Cu") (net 6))
 (segment (start 149.191553 94.508446) (end 149.191553 95.2) (width 0.17) (layer "F.Cu") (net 6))
 (segment (start 149.412691 94.33895) (end 149.380094 94.350356) (width 0.17) (layer "F.Cu") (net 6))
 (segment (start 149.380094 94.350356) (end 149.311458 94.358089) (width 0.17) (layer "F.Cu") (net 6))
 (segment (start 149.311458 94.358089) (end 149.278861 94.369495) (width 0.17) (layer "F.Cu") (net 6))
 (segment (start 149.484727 95.441531) (end 149.496133 95.474128) (width 0.17) (layer "F.Cu") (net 6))
 (segment (start 149.249619 94.387869) (end 149.225199 94.412289) (width 0.17) (layer "F.Cu") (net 6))
 (segment (start 149.412691 95.369495) (end 149.441933 95.387869) (width 0.17) (layer "F.Cu") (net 6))
 (segment (start 149.441933 95.387869) (end 149.466353 95.412289) (width 0.17) (layer "F.Cu") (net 6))
 (segment (start 149.466353 95.412289) (end 149.484727 95.441531) (width 0.17) (layer "F.Cu") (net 6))
 (segment (start 149.496133 95.474128) (end 149.5 95.508446) (width 0.17) (layer "F.Cu") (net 6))
 (segment (start 149.5 95.508446) (end 149.5 115.515198) (width 0.17) (layer "F.Cu") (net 6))
 (segment (start 149.5 115.515198) (end 148.595 116.420198) (width 0.17) (layer "F.Cu") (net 6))
 (segment (start 148.595 116.420198) (end 148.595 117.490168) (width 0.17) (layer "F.Cu") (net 6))
 (segment (start 148.595 117.490168) (end 148.595 119.37) (width 0.17) (layer "F.Cu") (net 6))
 (segment (start 148.05 95.75) (end 148.75 95.75) (width 0.17) (layer "F.Cu") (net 7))
 (segment (start 149.091225 96.477882) (end 149.06534 96.551859) (width 0.17) (layer "F.Cu") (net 7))
 (segment (start 147.776358 95.618221) (end 147.831778 95.673641) (width 0.17) (layer "F.Cu") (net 7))
 (segment (start 149.091225 96.022117) (end 149.1 96.1) (width 0.17) (layer "F.Cu") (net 7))
 (segment (start 148.90186 96.715339) (end 148.827883 96.741224) (width 0.17) (layer "F.Cu") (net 7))
 (segment (start 147.708775 95.477882) (end 147.73466 95.551859) (width 0.17) (layer "F.Cu") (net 7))
 (segment (start 147.7 95.4) (end 147.708775 95.477882) (width 0.17) (layer "F.Cu") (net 7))
 (segment (start 147.7 95.1) (end 147.7 95.4) (width 0.17) (layer "F.Cu") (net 7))
 (segment (start 147.776358 94.881778) (end 147.73466 94.94814) (width 0.17) (layer "F.Cu") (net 7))
 (segment (start 147.708775 95.022117) (end 147.7 95.1) (width 0.17) (layer "F.Cu") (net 7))
 (segment (start 149.1 96.4) (end 149.091225 96.477882) (width 0.17) (layer "F.Cu") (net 7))
 (segment (start 147.972117 95.741224) (end 148.05 95.75) (width 0.17) (layer "F.Cu") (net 7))
 (segment (start 148.365339 94.551859) (end 148.323641 94.618221) (width 0.17) (layer "F.Cu") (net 7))
 (segment (start 148.4 94.4) (end 148.391224 94.477882) (width 0.17) (layer "F.Cu") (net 7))
 (segment (start 148.90186 95.78466) (end 148.968222 95.826358) (width 0.17) (layer "F.Cu") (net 7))
 (segment (start 149.06534 95.94814) (end 149.091225 96.022117) (width 0.17) (layer "F.Cu") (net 7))
 (segment (start 147.73466 94.94814) (end 147.708775 95.022117) (width 0.17) (layer "F.Cu") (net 7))
 (segment (start 148.4 115.755) (end 147.325 116.83) (width 0.17) (layer "F.Cu") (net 7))
 (segment (start 148.268221 94.673641) (end 148.201859 94.715339) (width 0.17) (layer "F.Cu") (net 7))
 (segment (start 148.127882 94.741224) (end 147.972117 94.758775) (width 0.17) (layer "F.Cu") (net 7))
 (segment (start 147.73466 95.551859) (end 147.776358 95.618221) (width 0.17) (layer "F.Cu") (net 7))
 (segment (start 148.4 92.6) (end 148.4 94.4) (width 0.17) (layer "F.Cu") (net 7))
 (segment (start 148.4 97.1) (end 148.4 115.755) (width 0.17) (layer "F.Cu") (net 7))
 (segment (start 148.391224 94.477882) (end 148.365339 94.551859) (width 0.17) (layer "F.Cu") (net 7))
 (segment (start 148.201859 94.715339) (end 148.127882 94.741224) (width 0.17) (layer "F.Cu") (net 7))
 (segment (start 147.831778 95.673641) (end 147.89814 95.715339) (width 0.17) (layer "F.Cu") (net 7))
 (segment (start 148.323641 94.618221) (end 148.268221 94.673641) (width 0.17) (layer "F.Cu") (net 7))
 (segment (start 147.972117 94.758775) (end 147.89814 94.78466) (width 0.17) (layer "F.Cu") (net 7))
 (segment (start 148.531779 96.826358) (end 148.476359 96.881778) (width 0.17) (layer "F.Cu") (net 7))
 (segment (start 147.89814 94.78466) (end 147.831778 94.826358) (width 0.17) (layer "F.Cu") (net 7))
 (segment (start 147.89814 95.715339) (end 147.972117 95.741224) (width 0.17) (layer "F.Cu") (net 7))
 (segment (start 147.831778 94.826358) (end 147.776358 94.881778) (width 0.17) (layer "F.Cu") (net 7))
 (segment (start 148.476359 96.881778) (end 148.434661 96.94814) (width 0.17) (layer "F.Cu") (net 7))
 (segment (start 148.75 95.75) (end 148.827883 95.758775) (width 0.17) (layer "F.Cu") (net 7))
 (segment (start 148.827883 96.741224) (end 148.672118 96.758775) (width 0.17) (layer "F.Cu") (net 7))
 (segment (start 148.827883 95.758775) (end 148.90186 95.78466) (width 0.17) (layer "F.Cu") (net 7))
 (segment (start 148.968222 95.826358) (end 149.023642 95.881778) (width 0.17) (layer "F.Cu") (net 7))
 (segment (start 149.023642 95.881778) (end 149.06534 95.94814) (width 0.17) (layer "F.Cu") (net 7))
 (segment (start 149.1 96.1) (end 149.1 96.4) (width 0.17) (layer "F.Cu") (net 7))
 (segment (start 149.06534 96.551859) (end 149.023642 96.618221) (width 0.17) (layer "F.Cu") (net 7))
 (segment (start 149.023642 96.618221) (end 148.968222 96.673641) (width 0.17) (layer "F.Cu") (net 7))
 (segment (start 148.968222 96.673641) (end 148.90186 96.715339) (width 0.17) (layer "F.Cu") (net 7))
 (segment (start 148.672118 96.758775) (end 148.598141 96.78466) (width 0.17) (layer "F.Cu") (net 7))
 (segment (start 148.408776 97.022117) (end 148.4 97.1) (width 0.17) (layer "F.Cu") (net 7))
 (segment (start 148.598141 96.78466) (end 148.531779 96.826358) (width 0.17) (layer "F.Cu") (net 7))
 (segment (start 148.434661 96.94814) (end 148.408776 97.022117) (width 0.17) (layer "F.Cu") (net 7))
 (segment (start 146.055 116.420198) (end 147.3 115.175198) (width 0.17) (layer "F.Cu") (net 8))
 (segment (start 146.055 119.37) (end 146.055 116.420198) (width 0.17) (layer "F.Cu") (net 8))
 (segment (start 147.3 98.2) (end 147.3 92.6) (width 0.17) (layer "F.Cu") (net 8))
 (segment (start 147.3 115.175198) (end 147.3 98.2) (width 0.17) (layer "F.Cu") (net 8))
 (segment (start 152.8 92.4) (end 152.8 116.435) (width 0.25) (layer "F.Cu") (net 3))
 (segment (start 152.8 116.435) (end 152.405 116.83) (width 0.25) (layer "F.Cu") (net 3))
 (segment (start 150.6 92.4) (end 150.6 116.095) (width 0.25) (layer "F.Cu") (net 5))
 (segment (start 150.6 116.095) (end 149.865 116.83) (width 0.25) (layer "F.Cu") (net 5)))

